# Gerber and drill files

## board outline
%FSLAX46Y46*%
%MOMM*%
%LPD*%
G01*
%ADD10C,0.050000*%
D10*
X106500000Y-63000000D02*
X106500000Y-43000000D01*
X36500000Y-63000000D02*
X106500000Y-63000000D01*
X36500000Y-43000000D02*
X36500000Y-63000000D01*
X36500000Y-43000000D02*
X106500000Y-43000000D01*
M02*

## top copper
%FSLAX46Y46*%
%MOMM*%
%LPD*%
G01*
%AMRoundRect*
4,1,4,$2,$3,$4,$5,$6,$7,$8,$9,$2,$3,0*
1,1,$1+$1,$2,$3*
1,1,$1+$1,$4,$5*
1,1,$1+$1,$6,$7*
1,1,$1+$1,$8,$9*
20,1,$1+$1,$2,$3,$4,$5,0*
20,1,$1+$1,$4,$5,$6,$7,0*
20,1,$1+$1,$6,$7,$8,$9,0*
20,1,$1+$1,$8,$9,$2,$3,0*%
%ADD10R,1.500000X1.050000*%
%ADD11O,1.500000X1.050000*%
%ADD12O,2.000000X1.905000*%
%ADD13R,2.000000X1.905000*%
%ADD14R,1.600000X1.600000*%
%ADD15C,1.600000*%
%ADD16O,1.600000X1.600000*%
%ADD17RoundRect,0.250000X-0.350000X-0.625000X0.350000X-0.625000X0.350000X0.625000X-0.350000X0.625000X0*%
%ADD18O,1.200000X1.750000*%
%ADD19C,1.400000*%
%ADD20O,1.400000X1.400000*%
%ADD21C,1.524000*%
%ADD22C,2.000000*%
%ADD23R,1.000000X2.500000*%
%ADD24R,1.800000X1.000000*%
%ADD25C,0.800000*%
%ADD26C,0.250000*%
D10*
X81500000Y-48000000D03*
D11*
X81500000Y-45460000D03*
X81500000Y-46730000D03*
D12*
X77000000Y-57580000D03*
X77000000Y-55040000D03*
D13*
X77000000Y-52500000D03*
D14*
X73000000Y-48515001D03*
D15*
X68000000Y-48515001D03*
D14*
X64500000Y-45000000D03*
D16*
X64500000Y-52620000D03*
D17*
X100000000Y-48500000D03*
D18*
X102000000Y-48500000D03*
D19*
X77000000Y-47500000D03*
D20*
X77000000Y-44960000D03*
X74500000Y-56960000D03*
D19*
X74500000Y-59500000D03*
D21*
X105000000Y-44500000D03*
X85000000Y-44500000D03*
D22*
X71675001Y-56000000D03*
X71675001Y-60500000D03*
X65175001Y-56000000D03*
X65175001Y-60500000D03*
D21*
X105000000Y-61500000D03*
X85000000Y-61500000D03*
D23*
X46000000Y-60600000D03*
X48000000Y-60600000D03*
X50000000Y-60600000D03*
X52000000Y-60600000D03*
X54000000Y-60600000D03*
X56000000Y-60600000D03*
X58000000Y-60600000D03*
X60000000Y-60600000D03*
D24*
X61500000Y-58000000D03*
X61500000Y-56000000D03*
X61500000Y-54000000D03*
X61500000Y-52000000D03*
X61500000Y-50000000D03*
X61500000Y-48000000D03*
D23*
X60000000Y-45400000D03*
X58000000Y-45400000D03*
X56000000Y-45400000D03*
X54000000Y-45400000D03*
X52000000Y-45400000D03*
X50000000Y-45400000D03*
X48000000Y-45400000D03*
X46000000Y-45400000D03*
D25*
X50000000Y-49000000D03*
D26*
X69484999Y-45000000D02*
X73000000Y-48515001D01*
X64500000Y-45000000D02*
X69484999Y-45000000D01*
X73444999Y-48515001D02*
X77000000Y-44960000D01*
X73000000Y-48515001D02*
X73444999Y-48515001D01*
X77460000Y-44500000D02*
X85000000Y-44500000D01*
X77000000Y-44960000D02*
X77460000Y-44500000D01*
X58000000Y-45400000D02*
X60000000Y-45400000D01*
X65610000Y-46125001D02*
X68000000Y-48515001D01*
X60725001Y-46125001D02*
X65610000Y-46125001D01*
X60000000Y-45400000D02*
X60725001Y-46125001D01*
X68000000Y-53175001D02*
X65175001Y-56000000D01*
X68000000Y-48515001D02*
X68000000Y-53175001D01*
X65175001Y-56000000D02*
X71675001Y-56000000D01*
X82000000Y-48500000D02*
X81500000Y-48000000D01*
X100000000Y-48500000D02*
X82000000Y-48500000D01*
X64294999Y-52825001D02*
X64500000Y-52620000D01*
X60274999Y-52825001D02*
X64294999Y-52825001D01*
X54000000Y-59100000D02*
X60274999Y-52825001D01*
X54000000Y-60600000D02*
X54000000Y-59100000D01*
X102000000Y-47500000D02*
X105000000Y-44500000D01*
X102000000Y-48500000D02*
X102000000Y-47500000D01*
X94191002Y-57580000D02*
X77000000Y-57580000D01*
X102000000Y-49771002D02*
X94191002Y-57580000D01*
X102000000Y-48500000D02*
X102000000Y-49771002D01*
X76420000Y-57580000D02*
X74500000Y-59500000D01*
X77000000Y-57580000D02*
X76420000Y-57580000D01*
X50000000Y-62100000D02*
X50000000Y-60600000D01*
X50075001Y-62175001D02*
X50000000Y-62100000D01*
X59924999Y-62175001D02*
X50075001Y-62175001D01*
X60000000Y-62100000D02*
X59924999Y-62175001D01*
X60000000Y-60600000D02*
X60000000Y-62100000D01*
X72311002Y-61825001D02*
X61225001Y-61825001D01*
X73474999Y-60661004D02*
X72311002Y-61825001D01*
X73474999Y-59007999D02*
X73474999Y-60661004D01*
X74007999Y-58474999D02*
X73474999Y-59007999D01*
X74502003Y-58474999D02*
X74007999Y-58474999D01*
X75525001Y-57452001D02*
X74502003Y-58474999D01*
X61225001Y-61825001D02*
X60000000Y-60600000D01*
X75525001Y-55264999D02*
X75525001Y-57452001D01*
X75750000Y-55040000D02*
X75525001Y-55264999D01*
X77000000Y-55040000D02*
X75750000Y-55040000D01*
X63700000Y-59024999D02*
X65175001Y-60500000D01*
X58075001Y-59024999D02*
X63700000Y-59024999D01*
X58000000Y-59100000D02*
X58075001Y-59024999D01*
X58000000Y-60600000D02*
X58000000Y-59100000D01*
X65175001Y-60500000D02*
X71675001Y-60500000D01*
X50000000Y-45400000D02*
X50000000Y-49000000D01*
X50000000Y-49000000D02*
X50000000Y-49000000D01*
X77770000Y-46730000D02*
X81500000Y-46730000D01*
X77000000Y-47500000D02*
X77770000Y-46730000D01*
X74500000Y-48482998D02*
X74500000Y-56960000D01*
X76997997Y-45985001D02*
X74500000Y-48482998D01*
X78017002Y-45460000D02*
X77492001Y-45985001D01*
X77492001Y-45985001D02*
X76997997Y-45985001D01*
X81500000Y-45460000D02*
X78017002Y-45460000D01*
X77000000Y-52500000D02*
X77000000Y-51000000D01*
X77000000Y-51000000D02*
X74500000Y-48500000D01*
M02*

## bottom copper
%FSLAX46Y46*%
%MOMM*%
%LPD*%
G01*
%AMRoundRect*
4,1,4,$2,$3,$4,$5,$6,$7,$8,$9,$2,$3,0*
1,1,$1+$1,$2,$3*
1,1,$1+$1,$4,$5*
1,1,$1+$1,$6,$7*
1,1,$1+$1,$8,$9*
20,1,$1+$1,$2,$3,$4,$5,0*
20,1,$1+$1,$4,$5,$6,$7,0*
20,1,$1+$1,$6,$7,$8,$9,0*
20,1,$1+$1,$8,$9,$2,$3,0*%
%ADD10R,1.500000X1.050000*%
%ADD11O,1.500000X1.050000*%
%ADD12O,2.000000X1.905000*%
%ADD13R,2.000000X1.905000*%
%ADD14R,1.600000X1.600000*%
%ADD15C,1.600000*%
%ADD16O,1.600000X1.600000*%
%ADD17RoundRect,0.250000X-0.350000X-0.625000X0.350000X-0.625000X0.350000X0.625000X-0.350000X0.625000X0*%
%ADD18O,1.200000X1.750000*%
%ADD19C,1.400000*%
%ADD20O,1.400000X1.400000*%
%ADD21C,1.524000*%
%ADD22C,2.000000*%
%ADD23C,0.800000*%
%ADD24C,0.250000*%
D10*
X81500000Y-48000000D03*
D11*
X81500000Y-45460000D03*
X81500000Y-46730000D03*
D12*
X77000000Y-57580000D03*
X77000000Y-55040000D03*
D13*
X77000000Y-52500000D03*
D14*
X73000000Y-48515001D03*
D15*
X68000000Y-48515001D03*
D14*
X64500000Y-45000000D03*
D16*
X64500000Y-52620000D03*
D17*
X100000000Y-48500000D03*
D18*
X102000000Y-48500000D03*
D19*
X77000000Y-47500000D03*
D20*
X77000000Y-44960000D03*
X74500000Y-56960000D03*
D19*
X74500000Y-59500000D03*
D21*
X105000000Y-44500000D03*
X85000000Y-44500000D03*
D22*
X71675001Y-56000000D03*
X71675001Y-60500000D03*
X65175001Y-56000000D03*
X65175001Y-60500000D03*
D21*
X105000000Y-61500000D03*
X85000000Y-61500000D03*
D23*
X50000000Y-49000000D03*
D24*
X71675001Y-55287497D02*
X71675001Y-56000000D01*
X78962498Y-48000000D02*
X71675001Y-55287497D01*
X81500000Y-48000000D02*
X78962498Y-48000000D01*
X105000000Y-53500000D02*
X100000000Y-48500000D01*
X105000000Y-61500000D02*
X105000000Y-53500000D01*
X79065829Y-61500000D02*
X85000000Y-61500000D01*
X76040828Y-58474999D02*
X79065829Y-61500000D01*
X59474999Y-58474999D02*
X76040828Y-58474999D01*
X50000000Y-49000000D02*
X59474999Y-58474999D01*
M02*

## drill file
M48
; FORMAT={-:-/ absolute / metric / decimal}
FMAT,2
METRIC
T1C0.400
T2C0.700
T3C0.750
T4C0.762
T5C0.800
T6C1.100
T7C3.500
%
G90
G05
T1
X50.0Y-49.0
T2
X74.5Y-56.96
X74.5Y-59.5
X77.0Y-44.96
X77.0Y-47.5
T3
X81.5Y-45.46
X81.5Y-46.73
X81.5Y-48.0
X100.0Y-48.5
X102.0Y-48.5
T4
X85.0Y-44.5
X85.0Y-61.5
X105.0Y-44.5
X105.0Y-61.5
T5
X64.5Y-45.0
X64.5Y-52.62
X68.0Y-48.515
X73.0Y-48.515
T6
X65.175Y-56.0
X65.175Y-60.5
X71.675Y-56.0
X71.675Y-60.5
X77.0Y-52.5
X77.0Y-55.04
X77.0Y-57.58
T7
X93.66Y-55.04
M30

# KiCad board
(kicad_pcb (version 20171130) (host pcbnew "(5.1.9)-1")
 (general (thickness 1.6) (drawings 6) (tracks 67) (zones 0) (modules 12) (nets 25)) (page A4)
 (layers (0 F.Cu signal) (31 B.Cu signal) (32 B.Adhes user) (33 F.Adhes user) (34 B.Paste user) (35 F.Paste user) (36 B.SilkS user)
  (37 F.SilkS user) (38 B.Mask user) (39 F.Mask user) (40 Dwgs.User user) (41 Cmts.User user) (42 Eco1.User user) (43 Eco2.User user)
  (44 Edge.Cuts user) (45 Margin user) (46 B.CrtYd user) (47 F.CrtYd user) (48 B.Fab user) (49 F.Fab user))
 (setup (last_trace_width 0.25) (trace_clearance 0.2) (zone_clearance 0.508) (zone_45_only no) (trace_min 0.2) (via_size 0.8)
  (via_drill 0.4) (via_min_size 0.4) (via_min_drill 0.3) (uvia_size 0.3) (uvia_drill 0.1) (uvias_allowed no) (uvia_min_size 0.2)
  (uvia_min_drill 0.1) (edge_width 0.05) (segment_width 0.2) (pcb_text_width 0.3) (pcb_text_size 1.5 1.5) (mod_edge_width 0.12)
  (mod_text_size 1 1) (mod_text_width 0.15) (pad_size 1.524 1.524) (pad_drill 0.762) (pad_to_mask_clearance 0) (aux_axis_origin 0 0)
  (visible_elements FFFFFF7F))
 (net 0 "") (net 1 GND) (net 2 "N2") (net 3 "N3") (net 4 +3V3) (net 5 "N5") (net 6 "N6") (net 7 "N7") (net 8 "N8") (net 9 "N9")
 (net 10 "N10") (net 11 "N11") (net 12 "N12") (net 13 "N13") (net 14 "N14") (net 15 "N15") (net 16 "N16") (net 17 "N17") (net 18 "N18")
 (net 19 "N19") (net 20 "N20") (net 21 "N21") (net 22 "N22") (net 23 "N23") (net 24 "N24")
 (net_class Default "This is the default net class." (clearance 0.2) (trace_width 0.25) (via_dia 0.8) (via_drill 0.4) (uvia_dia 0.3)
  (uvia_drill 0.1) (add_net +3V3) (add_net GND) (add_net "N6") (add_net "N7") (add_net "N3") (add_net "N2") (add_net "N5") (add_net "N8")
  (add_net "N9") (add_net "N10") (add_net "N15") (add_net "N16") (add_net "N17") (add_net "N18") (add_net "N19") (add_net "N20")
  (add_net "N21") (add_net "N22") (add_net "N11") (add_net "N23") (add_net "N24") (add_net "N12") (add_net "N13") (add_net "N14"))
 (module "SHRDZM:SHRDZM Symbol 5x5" (layer F.Cu) (at 101 59.5)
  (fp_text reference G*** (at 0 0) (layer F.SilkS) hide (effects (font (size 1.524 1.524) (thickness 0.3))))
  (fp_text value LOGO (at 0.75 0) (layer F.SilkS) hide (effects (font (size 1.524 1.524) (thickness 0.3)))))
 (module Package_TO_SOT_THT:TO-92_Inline (layer F.Cu) (at 81.5 48 90)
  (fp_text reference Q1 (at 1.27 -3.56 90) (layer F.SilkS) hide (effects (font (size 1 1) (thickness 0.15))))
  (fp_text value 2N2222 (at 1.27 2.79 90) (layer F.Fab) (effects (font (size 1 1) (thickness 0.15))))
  (pad 1 thru_hole rect (at 0 0 90) (size 1.05 1.5) (drill 0.75) (layers *.Cu *.Mask) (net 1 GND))
  (pad 3 thru_hole oval (at 2.54 0 90) (size 1.05 1.5) (drill 0.75) (layers *.Cu *.Mask) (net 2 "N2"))
  (pad 2 thru_hole oval (at 1.27 0 90) (size 1.05 1.5) (drill 0.75) (layers *.Cu *.Mask) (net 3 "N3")))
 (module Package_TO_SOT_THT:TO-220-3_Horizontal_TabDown (layer F.Cu) (at 77 52.5 270)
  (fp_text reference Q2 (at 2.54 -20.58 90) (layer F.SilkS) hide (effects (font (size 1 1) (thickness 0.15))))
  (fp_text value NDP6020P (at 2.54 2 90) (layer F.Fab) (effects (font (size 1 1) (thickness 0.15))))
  (pad 3 thru_hole oval (at 5.08 0 270) (size 1.905 2) (drill 1.1) (layers *.Cu *.Mask) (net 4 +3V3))
  (pad 2 thru_hole oval (at 2.54 0 270) (size 1.905 2) (drill 1.1) (layers *.Cu *.Mask) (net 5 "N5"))
  (pad 1 thru_hole rect (at 0 0 270) (size 1.905 2) (drill 1.1) (layers *.Cu *.Mask) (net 2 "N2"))
  (pad "" np_thru_hole oval (at 2.54 -16.66 270) (size 3.5 3.5) (drill 3.5) (layers *.Cu *.Mask)))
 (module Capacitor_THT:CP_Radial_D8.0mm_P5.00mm (layer F.Cu) (at 73 48.515001 180)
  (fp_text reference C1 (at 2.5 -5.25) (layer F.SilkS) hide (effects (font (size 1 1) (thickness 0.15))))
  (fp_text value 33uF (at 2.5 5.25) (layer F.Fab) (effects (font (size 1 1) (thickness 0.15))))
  (pad 1 thru_hole rect (at 0 0 180) (size 1.6 1.6) (drill 0.8) (layers *.Cu *.Mask) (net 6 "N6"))
  (pad 2 thru_hole circle (at 5 0 180) (size 1.6 1.6) (drill 0.8) (layers *.Cu *.Mask) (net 1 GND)))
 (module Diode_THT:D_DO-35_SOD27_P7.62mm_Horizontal (layer F.Cu) (at 64.5 45 270)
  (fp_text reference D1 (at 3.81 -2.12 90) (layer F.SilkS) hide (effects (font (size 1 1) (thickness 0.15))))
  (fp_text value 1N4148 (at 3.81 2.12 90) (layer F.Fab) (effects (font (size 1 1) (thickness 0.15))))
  (pad 1 thru_hole rect (at 0 0 270) (size 1.6 1.6) (drill 0.8) (layers *.Cu *.Mask) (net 6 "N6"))
  (pad 2 thru_hole oval (at 7.62 0 270) (size 1.6 1.6) (drill 0.8) (layers *.Cu *.Mask) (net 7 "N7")))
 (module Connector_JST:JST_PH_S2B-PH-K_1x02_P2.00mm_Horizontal (layer F.Cu) (at 100 48.5)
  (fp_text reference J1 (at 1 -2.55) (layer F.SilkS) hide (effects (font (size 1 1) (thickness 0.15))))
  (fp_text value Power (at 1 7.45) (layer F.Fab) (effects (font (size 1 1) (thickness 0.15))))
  (pad 1 thru_hole roundrect (at 0 0) (size 1.2 1.75) (drill 0.75) (layers *.Cu *.Mask) (roundrect_rratio 0.208333) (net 1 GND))
  (pad 2 thru_hole oval (at 2 0) (size 1.2 1.75) (drill 0.75) (layers *.Cu *.Mask) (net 4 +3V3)))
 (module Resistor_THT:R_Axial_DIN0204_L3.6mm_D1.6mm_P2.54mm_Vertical (layer F.Cu) (at 77 47.5 90)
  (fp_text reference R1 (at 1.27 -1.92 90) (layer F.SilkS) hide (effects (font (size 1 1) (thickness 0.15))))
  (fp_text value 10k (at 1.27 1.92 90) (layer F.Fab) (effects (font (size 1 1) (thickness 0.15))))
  (pad 1 thru_hole circle (at 0 0 90) (size 1.4 1.4) (drill 0.7) (layers *.Cu *.Mask) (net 3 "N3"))
  (pad 2 thru_hole oval (at 2.54 0 90) (size 1.4 1.4) (drill 0.7) (layers *.Cu *.Mask) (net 6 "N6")))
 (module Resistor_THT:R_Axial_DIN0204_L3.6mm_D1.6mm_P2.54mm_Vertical (layer F.Cu) (at 74.5 59.5 90)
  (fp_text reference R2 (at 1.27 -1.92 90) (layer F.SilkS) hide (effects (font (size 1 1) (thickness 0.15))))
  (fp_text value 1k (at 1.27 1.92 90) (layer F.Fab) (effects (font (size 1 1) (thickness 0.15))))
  (pad 2 thru_hole oval (at 2.54 0 90) (size 1.4 1.4) (drill 0.7) (layers *.Cu *.Mask) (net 2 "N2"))
  (pad 1 thru_hole circle (at 0 0 90) (size 1.4 1.4) (drill 0.7) (layers *.Cu *.Mask) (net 4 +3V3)))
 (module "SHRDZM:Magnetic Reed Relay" (layer F.Cu) (at 95 44.5 180)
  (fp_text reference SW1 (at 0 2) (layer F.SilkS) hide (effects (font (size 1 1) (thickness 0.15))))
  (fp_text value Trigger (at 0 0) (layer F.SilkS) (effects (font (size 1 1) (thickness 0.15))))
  (pad 1 thru_hole circle (at -10 0 180) (size 1.524 1.524) (drill 0.762) (layers *.Cu *.Mask) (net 4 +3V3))
  (pad 2 thru_hole circle (at 10 0 180) (size 1.524 1.524) (drill 0.762) (layers *.Cu *.Mask) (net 6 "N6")))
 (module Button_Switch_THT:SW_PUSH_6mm (layer F.Cu) (at 71.675001 60.5 180)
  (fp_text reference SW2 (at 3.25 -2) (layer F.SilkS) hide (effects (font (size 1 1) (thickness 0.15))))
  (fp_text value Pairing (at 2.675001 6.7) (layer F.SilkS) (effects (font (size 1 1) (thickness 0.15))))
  (pad 2 thru_hole circle (at 0 4.5 270) (size 2 2) (drill 1.1) (layers *.Cu *.Mask) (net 1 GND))
  (pad 1 thru_hole circle (at 0 0 270) (size 2 2) (drill 1.1) (layers *.Cu *.Mask) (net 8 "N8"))
  (pad 2 thru_hole circle (at 6.5 4.5 270) (size 2 2) (drill 1.1) (layers *.Cu *.Mask) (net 1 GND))
  (pad 1 thru_hole circle (at 6.5 0 270) (size 2 2) (drill 1.1) (layers *.Cu *.Mask) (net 8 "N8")))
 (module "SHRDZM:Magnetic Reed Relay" (layer B.Cu) (at 95 61.5)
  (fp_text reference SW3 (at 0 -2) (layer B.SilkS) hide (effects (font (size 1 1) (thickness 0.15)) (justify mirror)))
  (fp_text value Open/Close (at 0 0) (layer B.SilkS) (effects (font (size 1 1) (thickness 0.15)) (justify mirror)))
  (pad 2 thru_hole circle (at 10 0) (size 1.524 1.524) (drill 0.762) (layers *.Cu *.Mask) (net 1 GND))
  (pad 1 thru_hole circle (at -10 0) (size 1.524 1.524) (drill 0.762) (layers *.Cu *.Mask) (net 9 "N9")))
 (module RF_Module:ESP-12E (layer F.Cu) (at 49.5 53 90)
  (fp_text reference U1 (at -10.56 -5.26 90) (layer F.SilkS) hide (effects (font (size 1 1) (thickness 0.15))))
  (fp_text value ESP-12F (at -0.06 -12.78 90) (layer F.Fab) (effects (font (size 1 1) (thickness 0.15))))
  (pad 1 smd rect (at -7.6 -3.5 90) (size 2.5 1) (layers F.Cu F.Paste F.Mask) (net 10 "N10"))
  (pad 2 smd rect (at -7.6 -1.5 90) (size 2.5 1) (layers F.Cu F.Paste F.Mask) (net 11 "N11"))
  (pad 3 smd rect (at -7.6 0.5 90) (size 2.5 1) (layers F.Cu F.Paste F.Mask) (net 5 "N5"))
  (pad 4 smd rect (at -7.6 2.5 90) (size 2.5 1) (layers F.Cu F.Paste F.Mask) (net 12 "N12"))
  (pad 5 smd rect (at -7.6 4.5 90) (size 2.5 1) (layers F.Cu F.Paste F.Mask) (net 7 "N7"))
  (pad 6 smd rect (at -7.6 6.5 90) (size 2.5 1) (layers F.Cu F.Paste F.Mask) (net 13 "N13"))
  (pad 7 smd rect (at -7.6 8.5 90) (size 2.5 1) (layers F.Cu F.Paste F.Mask) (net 8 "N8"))
  (pad 8 smd rect (at -7.6 10.5 90) (size 2.5 1) (layers F.Cu F.Paste F.Mask) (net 5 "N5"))
  (pad 9 smd rect (at -5 12 90) (size 1 1.8) (layers F.Cu F.Paste F.Mask) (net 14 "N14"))
  (pad 10 smd rect (at -3 12 90) (size 1 1.8) (layers F.Cu F.Paste F.Mask) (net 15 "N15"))
  (pad 11 smd rect (at -1 12 90) (size 1 1.8) (layers F.Cu F.Paste F.Mask) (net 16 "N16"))
  (pad 12 smd rect (at 1 12 90) (size 1 1.8) (layers F.Cu F.Paste F.Mask) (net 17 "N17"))
  (pad 13 smd rect (at 3 12 90) (size 1 1.8) (layers F.Cu F.Paste F.Mask) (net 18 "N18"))
  (pad 14 smd rect (at 5 12 90) (size 1 1.8) (layers F.Cu F.Paste F.Mask) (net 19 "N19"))
  (pad 15 smd rect (at 7.6 10.5 90) (size 2.5 1) (layers F.Cu F.Paste F.Mask) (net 1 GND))
  (pad 16 smd rect (at 7.6 8.5 90) (size 2.5 1) (layers F.Cu F.Paste F.Mask) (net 1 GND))
  (pad 17 smd rect (at 7.6 6.5 90) (size 2.5 1) (layers F.Cu F.Paste F.Mask) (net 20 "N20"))
  (pad 18 smd rect (at 7.6 4.5 90) (size 2.5 1) (layers F.Cu F.Paste F.Mask) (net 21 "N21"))
  (pad 19 smd rect (at 7.6 2.5 90) (size 2.5 1) (layers F.Cu F.Paste F.Mask) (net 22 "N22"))
  (pad 20 smd rect (at 7.6 0.5 90) (size 2.5 1) (layers F.Cu F.Paste F.Mask) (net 9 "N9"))
  (pad 21 smd rect (at 7.6 -1.5 90) (size 2.5 1) (layers F.Cu F.Paste F.Mask) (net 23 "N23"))
  (pad 22 smd rect (at 7.6 -3.5 90) (size 2.5 1) (layers F.Cu F.Paste F.Mask) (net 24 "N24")))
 (gr_line (start 106.5 63) (end 106.5 43) (layer Edge.Cuts) (width 0.05))
 (gr_line (start 36.5 63) (end 106.5 63) (layer Edge.Cuts) (width 0.05))
 (gr_line (start 36.5 43) (end 36.5 63) (layer Edge.Cuts) (width 0.05))
 (gr_line (start 36.5 43) (end 106.5 43) (layer Edge.Cuts) (width 0.05))
 (segment (start 69.484999 45) (end 73 48.515001) (width 0.25) (layer F.Cu) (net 6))
 (segment (start 64.5 45) (end 69.484999 45) (width 0.25) (layer F.Cu) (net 6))
 (segment (start 73.444999 48.515001) (end 77 44.96) (width 0.25) (layer F.Cu) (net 6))
 (segment (start 73 48.515001) (end 73.444999 48.515001) (width 0.25) (layer F.Cu) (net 6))
 (segment (start 77.46 44.5) (end 85 44.5) (width 0.25) (layer F.Cu) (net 6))
 (segment (start 77 44.96) (end 77.46 44.5) (width 0.25) (layer F.Cu) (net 6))
 (segment (start 58 45.4) (end 60 45.4) (width 0.25) (layer F.Cu) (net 1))
 (segment (start 65.61 46.125001) (end 68 48.515001) (width 0.25) (layer F.Cu) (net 1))
 (segment (start 60.725001 46.125001) (end 65.61 46.125001) (width 0.25) (layer F.Cu) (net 1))
 (segment (start 60 45.4) (end 60.725001 46.125001) (width 0.25) (layer F.Cu) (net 1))
 (segment (start 68 53.175001) (end 65.175001 56) (width 0.25) (layer F.Cu) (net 1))
 (segment (start 68 48.515001) (end 68 53.175001) (width 0.25) (layer F.Cu) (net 1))
 (segment (start 65.175001 56) (end 71.675001 56) (width 0.25) (layer F.Cu) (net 1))
 (segment (start 71.675001 55.287497) (end 71.675001 56) (width 0.25) (layer B.Cu) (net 1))
 (segment (start 78.962498 48) (end 71.675001 55.287497) (width 0.25) (layer B.Cu) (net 1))
 (segment (start 81.5 48) (end 78.962498 48) (width 0.25) (layer B.Cu) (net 1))
 (segment (start 82 48.5) (end 81.5 48) (width 0.25) (layer F.Cu) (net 1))
 (segment (start 100 48.5) (end 82 48.5) (width 0.25) (layer F.Cu) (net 1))
 (segment (start 105 53.5) (end 100 48.5) (width 0.25) (layer B.Cu) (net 1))
 (segment (start 105 61.5) (end 105 53.5) (width 0.25) (layer B.Cu) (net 1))
 (segment (start 64.294999 52.825001) (end 64.5 52.62) (width 0.25) (layer F.Cu) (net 7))
 (segment (start 60.274999 52.825001) (end 64.294999 52.825001) (width 0.25) (layer F.Cu) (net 7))
 (segment (start 54 59.1) (end 60.274999 52.825001) (width 0.25) (layer F.Cu) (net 7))
 (segment (start 54 60.6) (end 54 59.1) (width 0.25) (layer F.Cu) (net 7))
 (segment (start 102 47.5) (end 105 44.5) (width 0.25) (layer F.Cu) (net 4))
 (segment (start 102 48.5) (end 102 47.5) (width 0.25) (layer F.Cu) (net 4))
 (segment (start 94.191002 57.58) (end 77 57.58) (width 0.25) (layer F.Cu) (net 4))
 (segment (start 102 49.771002) (end 94.191002 57.58) (width 0.25) (layer F.Cu) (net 4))
 (segment (start 102 48.5) (end 102 49.771002) (width 0.25) (layer F.Cu) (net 4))
 (segment (start 76.42 57.58) (end 74.5 59.5) (width 0.25) (layer F.Cu) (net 4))
 (segment (start 77 57.58) (end 76.42 57.58) (width 0.25) (layer F.Cu) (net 4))
 (segment (start 50 62.1) (end 50 60.6) (width 0.25) (layer F.Cu) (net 5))
 (segment (start 50.075001 62.175001) (end 50 62.1) (width 0.25) (layer F.Cu) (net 5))
 (segment (start 59.924999 62.175001) (end 50.075001 62.175001) (width 0.25) (layer F.Cu) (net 5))
 (segment (start 60 62.1) (end 59.924999 62.175001) (width 0.25) (layer F.Cu) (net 5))
 (segment (start 60 60.6) (end 60 62.1) (width 0.25) (layer F.Cu) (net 5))
 (segment (start 72.311002 61.825001) (end 61.225001 61.825001) (width 0.25) (layer F.Cu) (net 5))
 (segment (start 73.474999 60.661004) (end 72.311002 61.825001) (width 0.25) (layer F.Cu) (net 5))
 (segment (start 73.474999 59.007999) (end 73.474999 60.661004) (width 0.25) (layer F.Cu) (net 5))
 (segment (start 74.007999 58.474999) (end 73.474999 59.007999) (width 0.25) (layer F.Cu) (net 5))
 (segment (start 74.502003 58.474999) (end 74.007999 58.474999) (width 0.25) (layer F.Cu) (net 5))
 (segment (start 75.525001 57.452001) (end 74.502003 58.474999) (width 0.25) (layer F.Cu) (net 5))
 (segment (start 61.225001 61.825001) (end 60 60.6) (width 0.25) (layer F.Cu) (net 5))
 (segment (start 75.525001 55.264999) (end 75.525001 57.452001) (width 0.25) (layer F.Cu) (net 5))
 (segment (start 75.75 55.04) (end 75.525001 55.264999) (width 0.25) (layer F.Cu) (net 5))
 (segment (start 77 55.04) (end 75.75 55.04) (width 0.25) (layer F.Cu) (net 5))
 (segment (start 63.7 59.024999) (end 65.175001 60.5) (width 0.25) (layer F.Cu) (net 8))
 (segment (start 58.075001 59.024999) (end 63.7 59.024999) (width 0.25) (layer F.Cu) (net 8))
 (segment (start 58 59.1) (end 58.075001 59.024999) (width 0.25) (layer F.Cu) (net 8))
 (segment (start 58 60.6) (end 58 59.1) (width 0.25) (layer F.Cu) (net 8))
 (segment (start 65.175001 60.5) (end 71.675001 60.5) (width 0.25) (layer F.Cu) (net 8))
 (segment (start 50 45.4) (end 50 49) (width 0.25) (layer F.Cu) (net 9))
 (segment (start 50 49) (end 50 49) (width 0.25) (layer F.Cu) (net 9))
 (via (at 50 49) (size 0.8) (drill 0.4) (layers F.Cu B.Cu) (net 9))
 (segment (start 79.065829 61.5) (end 85 61.5) (width 0.25) (layer B.Cu) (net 9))
 (segment (start 76.040828 58.474999) (end 79.065829 61.5) (width 0.25) (layer B.Cu) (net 9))
 (segment (start 59.474999 58.474999) (end 76.040828 58.474999) (width 0.25) (layer B.Cu) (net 9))
 (segment (start 50 49) (end 59.474999 58.474999) (width 0.25) (layer B.Cu) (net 9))
 (segment (start 77.77 46.73) (end 81.5 46.73) (width 0.25) (layer F.Cu) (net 3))
 (segment (start 77 47.5) (end 77.77 46.73) (width 0.25) (layer F.Cu) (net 3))
 (segment (start 74.5 48.482998) (end 74.5 56.96) (width 0.25) (layer F.Cu) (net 2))
 (segment (start 76.997997 45.985001) (end 74.5 48.482998) (width 0.25) (layer F.Cu) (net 2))
 (segment (start 78.017002 45.46) (end 77.492001 45.985001) (width 0.25) (layer F.Cu) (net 2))
 (segment (start 77.492001 45.985001) (end 76.997997 45.985001) (width 0.25) (layer F.Cu) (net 2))
 (segment (start 81.5 45.46) (end 78.017002 45.46) (width 0.25) (layer F.Cu) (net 2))
 (segment (start 77 52.5) (end 77 51) (width 0.25) (layer F.Cu) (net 2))
 (segment (start 77 51) (end 74.5 48.5) (width 0.25) (layer F.Cu) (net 2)))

